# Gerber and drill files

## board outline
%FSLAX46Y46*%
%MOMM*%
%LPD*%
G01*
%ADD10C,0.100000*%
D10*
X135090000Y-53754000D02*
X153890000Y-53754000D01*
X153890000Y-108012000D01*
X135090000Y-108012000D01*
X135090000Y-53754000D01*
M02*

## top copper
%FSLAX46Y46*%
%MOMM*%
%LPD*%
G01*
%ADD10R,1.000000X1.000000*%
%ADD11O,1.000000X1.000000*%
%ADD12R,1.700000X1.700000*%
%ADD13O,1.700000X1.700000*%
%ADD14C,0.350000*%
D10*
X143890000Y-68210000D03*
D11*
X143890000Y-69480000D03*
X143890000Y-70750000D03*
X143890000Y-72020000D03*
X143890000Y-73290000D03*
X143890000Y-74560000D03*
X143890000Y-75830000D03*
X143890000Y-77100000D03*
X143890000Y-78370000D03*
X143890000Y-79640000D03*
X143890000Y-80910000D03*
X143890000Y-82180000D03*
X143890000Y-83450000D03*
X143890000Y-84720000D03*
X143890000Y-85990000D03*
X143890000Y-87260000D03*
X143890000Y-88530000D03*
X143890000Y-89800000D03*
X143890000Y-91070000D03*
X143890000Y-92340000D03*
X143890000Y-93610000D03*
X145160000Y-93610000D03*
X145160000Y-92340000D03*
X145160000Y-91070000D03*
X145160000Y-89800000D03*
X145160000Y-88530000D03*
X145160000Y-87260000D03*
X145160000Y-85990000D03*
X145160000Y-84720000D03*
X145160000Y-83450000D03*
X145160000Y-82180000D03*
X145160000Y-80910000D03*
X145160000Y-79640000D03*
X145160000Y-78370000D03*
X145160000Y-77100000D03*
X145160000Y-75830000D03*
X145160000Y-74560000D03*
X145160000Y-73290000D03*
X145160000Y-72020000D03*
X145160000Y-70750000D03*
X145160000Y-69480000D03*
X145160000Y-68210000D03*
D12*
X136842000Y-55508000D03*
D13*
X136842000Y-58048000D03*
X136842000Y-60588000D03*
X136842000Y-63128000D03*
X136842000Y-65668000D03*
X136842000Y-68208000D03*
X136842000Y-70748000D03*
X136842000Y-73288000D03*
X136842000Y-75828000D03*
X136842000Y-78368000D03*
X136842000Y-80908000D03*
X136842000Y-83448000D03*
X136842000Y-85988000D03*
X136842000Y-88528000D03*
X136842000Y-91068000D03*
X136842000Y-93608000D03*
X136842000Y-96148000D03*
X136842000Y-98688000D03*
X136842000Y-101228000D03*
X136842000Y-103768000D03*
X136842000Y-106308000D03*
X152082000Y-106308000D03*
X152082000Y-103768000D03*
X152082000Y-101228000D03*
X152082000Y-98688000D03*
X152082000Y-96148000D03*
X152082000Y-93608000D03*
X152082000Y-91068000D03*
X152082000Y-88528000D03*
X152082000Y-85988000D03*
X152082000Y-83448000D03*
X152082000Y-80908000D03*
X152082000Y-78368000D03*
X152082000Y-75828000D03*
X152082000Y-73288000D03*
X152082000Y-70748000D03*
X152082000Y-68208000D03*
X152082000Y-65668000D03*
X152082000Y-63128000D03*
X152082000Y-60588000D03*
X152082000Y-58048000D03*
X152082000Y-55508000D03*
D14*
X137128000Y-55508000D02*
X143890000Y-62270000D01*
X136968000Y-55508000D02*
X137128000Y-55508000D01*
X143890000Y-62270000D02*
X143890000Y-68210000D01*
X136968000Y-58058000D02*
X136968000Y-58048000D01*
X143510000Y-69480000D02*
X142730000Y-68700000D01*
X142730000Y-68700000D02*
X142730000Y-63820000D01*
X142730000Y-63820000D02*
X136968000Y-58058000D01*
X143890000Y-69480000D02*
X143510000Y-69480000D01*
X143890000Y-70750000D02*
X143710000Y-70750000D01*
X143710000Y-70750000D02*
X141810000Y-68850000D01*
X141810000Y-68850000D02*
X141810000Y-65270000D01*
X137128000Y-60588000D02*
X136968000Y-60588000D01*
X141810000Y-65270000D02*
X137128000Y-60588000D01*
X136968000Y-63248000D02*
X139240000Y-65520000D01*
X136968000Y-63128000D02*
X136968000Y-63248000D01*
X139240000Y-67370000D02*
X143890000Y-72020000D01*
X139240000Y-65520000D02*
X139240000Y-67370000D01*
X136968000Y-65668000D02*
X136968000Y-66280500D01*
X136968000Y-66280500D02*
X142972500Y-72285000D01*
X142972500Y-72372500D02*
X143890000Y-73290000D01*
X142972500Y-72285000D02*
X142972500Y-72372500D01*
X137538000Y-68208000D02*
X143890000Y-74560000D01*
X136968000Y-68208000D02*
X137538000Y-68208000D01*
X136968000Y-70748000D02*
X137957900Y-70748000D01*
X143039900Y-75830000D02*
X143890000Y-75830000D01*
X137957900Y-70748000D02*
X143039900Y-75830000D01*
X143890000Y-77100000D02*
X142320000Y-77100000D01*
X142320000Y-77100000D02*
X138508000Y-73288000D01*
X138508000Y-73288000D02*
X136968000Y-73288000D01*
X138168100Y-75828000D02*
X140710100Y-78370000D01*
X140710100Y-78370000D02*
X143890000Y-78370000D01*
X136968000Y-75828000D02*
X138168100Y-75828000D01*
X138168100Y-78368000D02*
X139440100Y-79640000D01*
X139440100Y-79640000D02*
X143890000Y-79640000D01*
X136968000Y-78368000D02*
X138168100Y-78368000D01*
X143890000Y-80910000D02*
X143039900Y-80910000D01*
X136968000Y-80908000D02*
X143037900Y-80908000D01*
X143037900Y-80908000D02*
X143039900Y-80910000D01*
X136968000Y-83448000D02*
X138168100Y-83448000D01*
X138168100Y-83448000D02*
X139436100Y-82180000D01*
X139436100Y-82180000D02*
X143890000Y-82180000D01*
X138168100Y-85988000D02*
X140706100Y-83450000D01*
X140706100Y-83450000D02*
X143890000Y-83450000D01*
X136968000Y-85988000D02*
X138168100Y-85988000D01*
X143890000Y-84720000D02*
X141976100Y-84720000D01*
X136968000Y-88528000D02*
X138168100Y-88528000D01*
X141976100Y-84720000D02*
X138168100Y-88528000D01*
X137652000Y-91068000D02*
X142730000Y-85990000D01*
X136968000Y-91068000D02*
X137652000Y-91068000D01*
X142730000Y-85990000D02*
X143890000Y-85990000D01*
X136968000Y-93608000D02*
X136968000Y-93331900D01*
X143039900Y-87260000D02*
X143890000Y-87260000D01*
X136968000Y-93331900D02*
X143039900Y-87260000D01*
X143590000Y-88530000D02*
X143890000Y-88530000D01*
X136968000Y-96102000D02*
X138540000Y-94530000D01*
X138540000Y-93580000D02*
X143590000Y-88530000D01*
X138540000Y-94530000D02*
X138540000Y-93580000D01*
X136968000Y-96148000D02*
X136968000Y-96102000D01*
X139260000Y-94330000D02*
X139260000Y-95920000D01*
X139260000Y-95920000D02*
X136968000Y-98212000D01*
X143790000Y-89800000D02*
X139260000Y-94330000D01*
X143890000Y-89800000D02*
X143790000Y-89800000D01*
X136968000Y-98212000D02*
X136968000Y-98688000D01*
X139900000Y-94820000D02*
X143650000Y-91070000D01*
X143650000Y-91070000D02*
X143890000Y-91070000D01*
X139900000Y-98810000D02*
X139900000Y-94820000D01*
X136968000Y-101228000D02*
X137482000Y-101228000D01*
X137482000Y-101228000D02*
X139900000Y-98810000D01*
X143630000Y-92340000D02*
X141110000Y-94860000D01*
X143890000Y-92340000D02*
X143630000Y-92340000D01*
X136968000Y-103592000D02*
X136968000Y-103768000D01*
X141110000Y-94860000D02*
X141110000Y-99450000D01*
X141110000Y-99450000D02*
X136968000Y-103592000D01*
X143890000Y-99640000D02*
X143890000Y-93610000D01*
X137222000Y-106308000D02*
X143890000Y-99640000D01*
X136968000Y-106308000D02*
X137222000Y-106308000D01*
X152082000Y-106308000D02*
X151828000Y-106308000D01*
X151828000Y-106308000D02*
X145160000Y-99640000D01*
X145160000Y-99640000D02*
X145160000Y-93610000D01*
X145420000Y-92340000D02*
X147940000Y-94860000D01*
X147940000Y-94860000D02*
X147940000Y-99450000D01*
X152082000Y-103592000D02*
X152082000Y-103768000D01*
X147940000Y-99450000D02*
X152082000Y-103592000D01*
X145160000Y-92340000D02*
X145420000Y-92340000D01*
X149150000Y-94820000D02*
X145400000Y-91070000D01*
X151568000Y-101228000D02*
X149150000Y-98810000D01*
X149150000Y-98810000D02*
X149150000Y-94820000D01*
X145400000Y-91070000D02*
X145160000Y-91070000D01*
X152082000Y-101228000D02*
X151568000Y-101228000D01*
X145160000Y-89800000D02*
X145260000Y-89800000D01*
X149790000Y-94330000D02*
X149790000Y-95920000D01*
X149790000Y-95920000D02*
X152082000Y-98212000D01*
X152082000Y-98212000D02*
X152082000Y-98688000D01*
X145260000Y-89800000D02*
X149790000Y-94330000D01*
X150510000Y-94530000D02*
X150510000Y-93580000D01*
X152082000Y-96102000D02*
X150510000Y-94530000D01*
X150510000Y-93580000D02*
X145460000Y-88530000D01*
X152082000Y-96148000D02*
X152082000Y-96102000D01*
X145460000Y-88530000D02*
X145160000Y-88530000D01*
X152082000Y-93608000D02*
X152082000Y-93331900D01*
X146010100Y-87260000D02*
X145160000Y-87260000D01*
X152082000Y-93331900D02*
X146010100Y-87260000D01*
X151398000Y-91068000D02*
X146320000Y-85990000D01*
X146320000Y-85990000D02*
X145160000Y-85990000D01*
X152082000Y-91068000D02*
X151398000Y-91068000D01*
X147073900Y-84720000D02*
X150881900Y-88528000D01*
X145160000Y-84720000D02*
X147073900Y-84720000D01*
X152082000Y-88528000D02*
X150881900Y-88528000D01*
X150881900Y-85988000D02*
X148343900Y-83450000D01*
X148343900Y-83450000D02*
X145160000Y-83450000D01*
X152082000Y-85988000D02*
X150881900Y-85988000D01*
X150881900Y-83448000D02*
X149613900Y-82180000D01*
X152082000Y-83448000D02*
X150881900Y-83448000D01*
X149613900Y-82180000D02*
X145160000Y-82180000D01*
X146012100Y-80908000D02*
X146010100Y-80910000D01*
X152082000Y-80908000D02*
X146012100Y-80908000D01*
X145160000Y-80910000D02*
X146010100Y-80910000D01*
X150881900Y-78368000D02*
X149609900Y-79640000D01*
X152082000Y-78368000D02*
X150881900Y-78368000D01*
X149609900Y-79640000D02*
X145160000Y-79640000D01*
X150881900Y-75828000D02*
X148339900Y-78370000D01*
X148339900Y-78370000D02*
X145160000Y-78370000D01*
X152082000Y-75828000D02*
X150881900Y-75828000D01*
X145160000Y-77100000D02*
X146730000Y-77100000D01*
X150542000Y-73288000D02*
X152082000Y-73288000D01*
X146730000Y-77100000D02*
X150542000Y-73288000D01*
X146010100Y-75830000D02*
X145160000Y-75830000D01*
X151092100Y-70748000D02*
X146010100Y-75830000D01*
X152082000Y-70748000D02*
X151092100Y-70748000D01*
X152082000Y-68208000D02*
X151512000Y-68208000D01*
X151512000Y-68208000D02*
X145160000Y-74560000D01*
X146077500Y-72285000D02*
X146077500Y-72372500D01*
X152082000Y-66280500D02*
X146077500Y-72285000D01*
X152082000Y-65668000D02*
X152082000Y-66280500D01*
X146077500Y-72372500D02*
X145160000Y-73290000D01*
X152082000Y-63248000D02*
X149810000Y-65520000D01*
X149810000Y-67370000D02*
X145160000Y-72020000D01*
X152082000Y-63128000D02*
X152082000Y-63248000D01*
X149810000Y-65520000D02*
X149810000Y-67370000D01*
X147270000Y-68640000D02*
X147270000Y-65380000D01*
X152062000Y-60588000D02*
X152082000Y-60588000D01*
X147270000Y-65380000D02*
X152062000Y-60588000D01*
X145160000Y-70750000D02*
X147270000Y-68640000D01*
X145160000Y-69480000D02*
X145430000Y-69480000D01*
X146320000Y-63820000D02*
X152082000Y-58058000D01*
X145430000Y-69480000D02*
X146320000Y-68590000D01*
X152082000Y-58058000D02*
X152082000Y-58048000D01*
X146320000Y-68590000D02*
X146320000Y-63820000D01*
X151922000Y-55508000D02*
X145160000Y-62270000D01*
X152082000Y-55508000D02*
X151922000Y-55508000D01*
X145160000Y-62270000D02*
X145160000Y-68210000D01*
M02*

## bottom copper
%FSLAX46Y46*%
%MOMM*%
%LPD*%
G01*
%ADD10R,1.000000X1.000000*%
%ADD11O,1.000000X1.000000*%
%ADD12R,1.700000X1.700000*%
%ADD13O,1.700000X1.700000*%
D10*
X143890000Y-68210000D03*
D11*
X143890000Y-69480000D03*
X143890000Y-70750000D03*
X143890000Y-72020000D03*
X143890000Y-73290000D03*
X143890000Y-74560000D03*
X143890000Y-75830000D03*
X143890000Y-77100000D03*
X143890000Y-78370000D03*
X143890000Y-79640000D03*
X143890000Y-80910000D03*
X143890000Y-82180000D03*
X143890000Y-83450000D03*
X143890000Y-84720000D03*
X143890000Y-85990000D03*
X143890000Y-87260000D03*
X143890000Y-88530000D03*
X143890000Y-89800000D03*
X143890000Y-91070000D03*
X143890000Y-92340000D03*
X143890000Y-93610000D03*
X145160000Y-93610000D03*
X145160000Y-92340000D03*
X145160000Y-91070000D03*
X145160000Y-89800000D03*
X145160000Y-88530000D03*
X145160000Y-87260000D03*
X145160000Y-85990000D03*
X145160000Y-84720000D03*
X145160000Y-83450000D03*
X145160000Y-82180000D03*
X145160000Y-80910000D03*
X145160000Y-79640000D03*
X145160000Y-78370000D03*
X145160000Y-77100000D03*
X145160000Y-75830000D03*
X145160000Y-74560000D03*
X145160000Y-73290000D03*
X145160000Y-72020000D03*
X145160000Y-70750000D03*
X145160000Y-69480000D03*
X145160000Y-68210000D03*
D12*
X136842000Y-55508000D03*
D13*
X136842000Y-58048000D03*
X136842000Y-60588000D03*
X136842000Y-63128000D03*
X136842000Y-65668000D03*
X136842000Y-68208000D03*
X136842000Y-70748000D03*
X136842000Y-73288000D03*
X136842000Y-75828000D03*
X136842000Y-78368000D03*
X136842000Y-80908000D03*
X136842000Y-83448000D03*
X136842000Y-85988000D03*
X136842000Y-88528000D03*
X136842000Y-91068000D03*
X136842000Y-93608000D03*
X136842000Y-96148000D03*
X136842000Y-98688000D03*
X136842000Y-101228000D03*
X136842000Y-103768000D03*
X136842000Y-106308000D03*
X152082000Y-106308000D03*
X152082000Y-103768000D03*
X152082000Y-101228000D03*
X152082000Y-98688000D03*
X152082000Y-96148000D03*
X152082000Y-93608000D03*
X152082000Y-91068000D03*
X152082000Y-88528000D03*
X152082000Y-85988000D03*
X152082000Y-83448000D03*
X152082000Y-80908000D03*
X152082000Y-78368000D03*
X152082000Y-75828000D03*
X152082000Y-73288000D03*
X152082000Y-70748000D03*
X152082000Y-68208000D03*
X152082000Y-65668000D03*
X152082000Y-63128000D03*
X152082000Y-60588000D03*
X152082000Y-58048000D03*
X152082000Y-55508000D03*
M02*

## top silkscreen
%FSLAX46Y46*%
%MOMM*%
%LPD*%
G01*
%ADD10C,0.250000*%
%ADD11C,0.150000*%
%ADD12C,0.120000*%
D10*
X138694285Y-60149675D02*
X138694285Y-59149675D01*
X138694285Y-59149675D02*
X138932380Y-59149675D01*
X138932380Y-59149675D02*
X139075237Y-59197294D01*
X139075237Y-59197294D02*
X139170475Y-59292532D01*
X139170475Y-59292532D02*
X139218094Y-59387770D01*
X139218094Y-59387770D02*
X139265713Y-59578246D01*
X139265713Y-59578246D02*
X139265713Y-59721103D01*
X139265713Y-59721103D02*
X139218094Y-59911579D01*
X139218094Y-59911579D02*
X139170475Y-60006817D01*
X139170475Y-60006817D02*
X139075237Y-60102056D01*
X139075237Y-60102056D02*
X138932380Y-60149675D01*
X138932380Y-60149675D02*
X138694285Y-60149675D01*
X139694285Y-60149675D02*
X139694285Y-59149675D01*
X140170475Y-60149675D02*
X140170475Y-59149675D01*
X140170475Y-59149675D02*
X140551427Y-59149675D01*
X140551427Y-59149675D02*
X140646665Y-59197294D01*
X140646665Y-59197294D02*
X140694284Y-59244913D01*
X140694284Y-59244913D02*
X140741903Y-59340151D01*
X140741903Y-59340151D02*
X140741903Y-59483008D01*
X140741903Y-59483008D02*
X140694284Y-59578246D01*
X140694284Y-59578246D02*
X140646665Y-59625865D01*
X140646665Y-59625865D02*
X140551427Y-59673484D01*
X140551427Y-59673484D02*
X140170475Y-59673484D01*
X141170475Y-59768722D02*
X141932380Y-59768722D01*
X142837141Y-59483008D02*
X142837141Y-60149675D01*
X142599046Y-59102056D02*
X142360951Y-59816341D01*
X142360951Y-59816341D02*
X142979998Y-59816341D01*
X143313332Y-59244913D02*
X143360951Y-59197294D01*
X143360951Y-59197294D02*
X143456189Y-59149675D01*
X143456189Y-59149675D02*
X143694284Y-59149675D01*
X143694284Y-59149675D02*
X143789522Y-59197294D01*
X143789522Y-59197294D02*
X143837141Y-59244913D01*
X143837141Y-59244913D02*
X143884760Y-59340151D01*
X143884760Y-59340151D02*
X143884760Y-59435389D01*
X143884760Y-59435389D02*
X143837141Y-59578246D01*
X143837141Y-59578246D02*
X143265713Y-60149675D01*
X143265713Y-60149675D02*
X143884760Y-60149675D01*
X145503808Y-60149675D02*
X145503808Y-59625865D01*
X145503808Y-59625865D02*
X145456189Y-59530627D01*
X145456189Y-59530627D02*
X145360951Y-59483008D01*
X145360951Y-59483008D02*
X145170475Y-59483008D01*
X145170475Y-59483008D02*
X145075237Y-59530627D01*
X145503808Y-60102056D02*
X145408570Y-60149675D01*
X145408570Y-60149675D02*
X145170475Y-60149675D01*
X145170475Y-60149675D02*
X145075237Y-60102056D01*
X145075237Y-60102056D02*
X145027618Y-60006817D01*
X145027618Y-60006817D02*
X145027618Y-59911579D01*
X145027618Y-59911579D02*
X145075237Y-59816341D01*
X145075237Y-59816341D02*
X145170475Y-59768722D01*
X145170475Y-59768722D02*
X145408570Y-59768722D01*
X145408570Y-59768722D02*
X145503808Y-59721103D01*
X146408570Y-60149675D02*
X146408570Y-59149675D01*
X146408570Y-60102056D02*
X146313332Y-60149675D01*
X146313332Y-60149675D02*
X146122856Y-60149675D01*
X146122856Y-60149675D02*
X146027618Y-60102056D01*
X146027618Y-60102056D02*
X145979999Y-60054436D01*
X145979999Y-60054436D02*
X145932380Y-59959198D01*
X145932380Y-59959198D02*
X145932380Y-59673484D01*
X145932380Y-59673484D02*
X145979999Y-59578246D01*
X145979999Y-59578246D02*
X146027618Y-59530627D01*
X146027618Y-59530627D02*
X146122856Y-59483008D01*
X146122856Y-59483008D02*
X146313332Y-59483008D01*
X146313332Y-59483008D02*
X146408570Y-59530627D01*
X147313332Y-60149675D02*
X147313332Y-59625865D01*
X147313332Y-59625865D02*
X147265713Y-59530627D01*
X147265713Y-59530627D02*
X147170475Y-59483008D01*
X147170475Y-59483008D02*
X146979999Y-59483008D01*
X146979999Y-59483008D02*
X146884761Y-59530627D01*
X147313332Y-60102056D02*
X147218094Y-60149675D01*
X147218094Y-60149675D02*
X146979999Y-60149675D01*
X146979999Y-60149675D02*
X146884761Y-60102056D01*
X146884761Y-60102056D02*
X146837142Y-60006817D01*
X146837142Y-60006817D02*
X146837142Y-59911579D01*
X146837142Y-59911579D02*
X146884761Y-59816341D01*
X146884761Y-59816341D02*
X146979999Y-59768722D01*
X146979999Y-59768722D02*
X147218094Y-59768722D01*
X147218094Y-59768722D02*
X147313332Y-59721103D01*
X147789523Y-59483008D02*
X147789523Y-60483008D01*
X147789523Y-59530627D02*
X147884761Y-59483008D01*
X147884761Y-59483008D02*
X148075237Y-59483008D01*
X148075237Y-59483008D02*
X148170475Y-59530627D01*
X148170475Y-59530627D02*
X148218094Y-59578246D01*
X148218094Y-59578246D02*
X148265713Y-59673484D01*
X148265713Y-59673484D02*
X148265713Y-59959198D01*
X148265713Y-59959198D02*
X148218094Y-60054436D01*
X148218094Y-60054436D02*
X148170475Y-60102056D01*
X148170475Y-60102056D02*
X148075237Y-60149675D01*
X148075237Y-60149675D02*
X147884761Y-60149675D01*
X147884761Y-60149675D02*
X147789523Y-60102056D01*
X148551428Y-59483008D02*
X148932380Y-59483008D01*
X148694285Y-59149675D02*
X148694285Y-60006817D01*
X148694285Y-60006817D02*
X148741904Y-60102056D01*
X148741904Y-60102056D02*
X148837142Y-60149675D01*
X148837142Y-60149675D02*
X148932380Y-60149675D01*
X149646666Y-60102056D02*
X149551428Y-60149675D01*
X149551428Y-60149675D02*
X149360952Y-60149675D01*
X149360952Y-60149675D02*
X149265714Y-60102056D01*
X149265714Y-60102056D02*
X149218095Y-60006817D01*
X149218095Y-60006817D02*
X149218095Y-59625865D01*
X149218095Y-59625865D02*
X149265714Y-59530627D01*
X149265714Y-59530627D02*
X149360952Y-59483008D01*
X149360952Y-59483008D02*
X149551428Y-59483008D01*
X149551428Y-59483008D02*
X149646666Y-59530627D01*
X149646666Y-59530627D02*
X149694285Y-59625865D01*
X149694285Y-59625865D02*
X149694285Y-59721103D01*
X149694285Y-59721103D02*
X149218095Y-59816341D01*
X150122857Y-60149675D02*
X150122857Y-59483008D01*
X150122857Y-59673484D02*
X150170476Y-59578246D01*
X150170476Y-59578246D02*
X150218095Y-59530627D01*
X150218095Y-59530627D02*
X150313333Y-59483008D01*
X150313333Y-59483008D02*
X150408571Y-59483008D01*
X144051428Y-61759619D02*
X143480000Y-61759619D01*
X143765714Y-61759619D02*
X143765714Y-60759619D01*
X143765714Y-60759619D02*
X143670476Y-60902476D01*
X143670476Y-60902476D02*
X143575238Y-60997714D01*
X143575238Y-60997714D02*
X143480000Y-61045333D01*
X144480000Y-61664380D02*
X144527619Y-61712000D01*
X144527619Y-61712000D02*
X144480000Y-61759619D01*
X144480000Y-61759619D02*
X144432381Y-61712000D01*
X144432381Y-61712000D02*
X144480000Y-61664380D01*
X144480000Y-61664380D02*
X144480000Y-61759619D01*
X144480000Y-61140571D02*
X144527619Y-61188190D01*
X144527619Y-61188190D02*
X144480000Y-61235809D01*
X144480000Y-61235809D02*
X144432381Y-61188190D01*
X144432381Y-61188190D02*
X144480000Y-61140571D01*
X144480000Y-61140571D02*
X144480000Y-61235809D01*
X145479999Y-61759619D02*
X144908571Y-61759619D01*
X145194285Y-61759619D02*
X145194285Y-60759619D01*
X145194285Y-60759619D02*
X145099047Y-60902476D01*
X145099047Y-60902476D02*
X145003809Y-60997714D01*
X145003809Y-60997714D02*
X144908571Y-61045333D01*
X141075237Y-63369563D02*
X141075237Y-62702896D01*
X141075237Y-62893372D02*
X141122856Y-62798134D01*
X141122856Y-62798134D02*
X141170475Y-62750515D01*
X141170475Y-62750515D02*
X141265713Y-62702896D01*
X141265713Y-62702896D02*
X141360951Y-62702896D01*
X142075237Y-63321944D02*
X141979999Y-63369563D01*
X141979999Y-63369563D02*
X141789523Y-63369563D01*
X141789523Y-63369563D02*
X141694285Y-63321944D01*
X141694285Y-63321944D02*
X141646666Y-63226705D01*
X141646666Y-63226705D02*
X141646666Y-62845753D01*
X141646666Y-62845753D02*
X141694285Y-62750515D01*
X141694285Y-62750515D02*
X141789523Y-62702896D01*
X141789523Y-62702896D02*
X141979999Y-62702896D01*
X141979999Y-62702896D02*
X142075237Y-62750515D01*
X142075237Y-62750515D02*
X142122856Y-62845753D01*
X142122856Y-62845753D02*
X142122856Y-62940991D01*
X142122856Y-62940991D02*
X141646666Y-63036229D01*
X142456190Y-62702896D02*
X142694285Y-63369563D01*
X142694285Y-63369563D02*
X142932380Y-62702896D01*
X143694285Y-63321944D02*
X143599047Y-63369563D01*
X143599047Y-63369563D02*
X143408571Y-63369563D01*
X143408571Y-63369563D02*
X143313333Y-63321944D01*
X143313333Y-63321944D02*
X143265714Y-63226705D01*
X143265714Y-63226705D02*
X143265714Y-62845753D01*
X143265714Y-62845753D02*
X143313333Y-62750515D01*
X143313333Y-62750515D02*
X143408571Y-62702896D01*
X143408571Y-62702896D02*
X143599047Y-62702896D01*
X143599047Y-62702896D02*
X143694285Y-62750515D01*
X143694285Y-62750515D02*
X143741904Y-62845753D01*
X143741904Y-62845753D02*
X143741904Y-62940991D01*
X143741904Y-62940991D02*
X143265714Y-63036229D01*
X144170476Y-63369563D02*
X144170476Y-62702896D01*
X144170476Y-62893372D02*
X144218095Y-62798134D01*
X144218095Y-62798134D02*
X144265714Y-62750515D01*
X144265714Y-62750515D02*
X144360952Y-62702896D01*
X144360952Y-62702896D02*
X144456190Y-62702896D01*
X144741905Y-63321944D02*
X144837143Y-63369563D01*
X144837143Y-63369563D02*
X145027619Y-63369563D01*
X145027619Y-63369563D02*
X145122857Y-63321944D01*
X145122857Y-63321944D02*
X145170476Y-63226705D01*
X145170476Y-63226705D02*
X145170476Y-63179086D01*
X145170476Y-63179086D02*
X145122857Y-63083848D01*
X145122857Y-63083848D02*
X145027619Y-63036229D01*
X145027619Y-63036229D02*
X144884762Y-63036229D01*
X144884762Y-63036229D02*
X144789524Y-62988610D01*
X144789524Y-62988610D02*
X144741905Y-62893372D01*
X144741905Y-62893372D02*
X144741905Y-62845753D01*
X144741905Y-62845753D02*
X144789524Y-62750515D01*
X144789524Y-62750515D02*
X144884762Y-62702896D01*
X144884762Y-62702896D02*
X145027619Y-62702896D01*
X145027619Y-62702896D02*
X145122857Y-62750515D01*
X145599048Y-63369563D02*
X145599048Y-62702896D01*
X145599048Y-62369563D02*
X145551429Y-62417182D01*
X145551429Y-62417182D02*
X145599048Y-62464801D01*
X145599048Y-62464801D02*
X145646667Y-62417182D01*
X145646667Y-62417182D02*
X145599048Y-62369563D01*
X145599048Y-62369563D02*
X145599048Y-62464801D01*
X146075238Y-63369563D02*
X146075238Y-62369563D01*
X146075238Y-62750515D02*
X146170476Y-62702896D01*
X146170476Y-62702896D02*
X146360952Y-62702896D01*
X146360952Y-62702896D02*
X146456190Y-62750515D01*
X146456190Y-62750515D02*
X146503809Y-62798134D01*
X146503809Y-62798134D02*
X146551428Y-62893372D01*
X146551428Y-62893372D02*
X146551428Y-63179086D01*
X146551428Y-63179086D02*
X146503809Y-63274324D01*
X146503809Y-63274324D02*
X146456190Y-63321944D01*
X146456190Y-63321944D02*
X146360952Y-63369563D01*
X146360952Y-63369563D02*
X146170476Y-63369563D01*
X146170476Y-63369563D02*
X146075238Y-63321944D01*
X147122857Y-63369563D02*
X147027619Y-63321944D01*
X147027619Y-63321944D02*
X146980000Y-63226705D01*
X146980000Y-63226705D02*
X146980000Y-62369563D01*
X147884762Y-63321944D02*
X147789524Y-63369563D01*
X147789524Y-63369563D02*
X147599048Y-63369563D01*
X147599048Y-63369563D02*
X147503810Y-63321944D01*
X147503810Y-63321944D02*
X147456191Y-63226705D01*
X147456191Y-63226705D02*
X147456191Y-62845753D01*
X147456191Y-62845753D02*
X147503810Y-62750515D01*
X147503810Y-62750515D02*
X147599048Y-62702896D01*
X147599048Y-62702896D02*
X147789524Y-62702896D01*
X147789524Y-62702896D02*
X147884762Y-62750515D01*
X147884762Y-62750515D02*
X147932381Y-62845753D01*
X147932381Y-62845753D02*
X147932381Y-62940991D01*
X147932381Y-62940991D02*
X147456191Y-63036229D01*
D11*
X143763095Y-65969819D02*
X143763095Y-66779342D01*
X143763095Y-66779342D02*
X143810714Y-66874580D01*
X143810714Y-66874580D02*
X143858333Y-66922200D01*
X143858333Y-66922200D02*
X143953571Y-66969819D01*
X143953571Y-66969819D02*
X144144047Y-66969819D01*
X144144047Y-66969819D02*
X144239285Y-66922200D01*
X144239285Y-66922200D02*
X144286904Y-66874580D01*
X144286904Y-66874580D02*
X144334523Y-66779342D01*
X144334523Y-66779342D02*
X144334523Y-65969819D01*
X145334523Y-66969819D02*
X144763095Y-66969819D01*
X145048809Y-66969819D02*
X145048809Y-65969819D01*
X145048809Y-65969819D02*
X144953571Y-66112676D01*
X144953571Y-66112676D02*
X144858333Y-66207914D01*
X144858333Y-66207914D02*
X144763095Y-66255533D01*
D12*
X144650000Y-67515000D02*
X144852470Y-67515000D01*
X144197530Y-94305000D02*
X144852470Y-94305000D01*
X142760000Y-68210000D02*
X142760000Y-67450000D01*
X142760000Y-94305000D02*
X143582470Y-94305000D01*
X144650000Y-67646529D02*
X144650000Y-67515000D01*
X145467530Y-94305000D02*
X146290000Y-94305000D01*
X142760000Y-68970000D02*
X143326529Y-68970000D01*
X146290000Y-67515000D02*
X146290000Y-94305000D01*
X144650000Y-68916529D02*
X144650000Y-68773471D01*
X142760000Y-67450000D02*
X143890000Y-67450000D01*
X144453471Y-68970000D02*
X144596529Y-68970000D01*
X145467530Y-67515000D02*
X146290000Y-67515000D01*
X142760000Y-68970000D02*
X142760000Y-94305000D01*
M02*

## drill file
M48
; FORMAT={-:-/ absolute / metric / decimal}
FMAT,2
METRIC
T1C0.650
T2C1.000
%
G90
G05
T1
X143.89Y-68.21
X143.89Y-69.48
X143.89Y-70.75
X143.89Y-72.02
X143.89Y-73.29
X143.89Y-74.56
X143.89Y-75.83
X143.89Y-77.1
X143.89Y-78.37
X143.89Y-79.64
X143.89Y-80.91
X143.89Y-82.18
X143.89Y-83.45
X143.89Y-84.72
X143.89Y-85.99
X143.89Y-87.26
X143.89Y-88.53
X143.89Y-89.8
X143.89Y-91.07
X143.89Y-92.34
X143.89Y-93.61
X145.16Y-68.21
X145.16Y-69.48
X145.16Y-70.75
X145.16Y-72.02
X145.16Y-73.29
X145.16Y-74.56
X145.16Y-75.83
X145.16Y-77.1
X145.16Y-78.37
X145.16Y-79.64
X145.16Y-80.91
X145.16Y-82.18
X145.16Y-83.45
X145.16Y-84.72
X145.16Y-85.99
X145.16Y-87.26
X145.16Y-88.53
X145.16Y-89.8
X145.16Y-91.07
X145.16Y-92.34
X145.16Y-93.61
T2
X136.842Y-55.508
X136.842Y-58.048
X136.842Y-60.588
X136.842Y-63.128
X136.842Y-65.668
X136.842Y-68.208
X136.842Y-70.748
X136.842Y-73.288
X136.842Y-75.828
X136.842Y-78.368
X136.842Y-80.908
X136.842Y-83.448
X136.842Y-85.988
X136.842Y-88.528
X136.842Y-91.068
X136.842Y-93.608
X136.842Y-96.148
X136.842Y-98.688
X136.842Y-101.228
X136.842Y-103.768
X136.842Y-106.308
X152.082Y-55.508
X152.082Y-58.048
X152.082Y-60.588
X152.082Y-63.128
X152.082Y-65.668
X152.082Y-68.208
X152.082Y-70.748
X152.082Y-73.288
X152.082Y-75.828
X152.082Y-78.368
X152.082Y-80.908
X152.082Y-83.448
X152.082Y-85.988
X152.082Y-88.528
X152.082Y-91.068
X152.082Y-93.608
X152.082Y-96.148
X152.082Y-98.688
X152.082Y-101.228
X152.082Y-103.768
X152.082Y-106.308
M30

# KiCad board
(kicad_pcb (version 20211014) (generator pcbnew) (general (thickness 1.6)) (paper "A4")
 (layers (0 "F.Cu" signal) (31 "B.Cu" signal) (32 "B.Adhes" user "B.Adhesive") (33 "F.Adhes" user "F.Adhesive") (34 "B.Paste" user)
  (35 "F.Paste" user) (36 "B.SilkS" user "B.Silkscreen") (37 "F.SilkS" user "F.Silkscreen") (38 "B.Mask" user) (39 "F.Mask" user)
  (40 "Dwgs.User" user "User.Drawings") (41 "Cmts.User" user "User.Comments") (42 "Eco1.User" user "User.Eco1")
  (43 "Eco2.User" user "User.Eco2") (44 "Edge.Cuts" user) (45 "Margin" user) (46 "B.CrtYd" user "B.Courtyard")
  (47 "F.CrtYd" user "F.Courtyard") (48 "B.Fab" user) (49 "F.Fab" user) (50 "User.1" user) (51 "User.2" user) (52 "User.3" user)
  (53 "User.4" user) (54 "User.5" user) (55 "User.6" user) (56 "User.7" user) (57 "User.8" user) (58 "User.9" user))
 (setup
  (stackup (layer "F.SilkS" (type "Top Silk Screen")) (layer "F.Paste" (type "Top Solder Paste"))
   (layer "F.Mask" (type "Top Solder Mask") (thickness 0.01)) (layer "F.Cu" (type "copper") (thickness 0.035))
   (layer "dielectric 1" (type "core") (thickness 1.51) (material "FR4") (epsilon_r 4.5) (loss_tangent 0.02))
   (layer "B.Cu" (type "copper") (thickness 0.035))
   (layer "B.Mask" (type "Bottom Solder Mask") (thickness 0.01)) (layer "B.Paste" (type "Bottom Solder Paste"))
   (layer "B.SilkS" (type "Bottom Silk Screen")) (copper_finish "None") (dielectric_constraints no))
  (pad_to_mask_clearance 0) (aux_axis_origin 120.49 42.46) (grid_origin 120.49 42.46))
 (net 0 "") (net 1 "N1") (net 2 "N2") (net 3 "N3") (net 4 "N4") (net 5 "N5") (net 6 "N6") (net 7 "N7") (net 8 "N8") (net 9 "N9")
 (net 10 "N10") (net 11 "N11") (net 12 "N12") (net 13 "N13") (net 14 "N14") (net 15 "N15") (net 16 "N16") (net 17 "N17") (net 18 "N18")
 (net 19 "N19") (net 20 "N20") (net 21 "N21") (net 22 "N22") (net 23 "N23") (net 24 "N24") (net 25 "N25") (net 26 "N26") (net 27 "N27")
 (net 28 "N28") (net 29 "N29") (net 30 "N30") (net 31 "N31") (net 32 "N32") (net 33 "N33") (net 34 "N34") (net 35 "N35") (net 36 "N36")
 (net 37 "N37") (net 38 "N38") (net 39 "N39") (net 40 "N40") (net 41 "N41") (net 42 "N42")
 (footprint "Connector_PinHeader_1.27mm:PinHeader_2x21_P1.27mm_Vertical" (layer "F.Cu") (at 143.89 68.21)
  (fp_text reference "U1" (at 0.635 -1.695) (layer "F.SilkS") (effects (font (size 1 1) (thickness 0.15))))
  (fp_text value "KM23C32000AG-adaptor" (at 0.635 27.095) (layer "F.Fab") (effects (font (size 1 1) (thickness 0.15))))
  (fp_line (start 0.76 -0.695) (end 0.96247 -0.695) (layer "F.SilkS") (width 0.12))
  (fp_line (start 0.30753 26.095) (end 0.96247 26.095) (layer "F.SilkS") (width 0.12))
  (fp_line (start -1.13 0) (end -1.13 -0.76) (layer "F.SilkS") (width 0.12))
  (fp_line (start -1.13 26.095) (end -0.30753 26.095) (layer "F.SilkS") (width 0.12))
  (fp_line (start 0.76 -0.563471) (end 0.76 -0.695) (layer "F.SilkS") (width 0.12))
  (fp_line (start 1.57753 26.095) (end 2.4 26.095) (layer "F.SilkS") (width 0.12))
  (fp_line (start -1.13 0.76) (end -0.563471 0.76) (layer "F.SilkS") (width 0.12))
  (fp_line (start 2.4 -0.695) (end 2.4 26.095) (layer "F.SilkS") (width 0.12))
  (fp_line (start 0.76 0.706529) (end 0.76 0.563471) (layer "F.SilkS") (width 0.12))
  (fp_line (start -1.13 -0.76) (end 0 -0.76) (layer "F.SilkS") (width 0.12))
  (fp_line (start 0.563471 0.76) (end 0.706529 0.76) (layer "F.SilkS") (width 0.12))
  (fp_line (start 1.57753 -0.695) (end 2.4 -0.695) (layer "F.SilkS") (width 0.12))
  (fp_line (start -1.13 0.76) (end -1.13 26.095) (layer "F.SilkS") (width 0.12))
  (pad "1" thru_hole rect (at 0 0) (size 1 1) (drill 0.65) (layers *.Cu *.Mask) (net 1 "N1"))
  (pad "2" thru_hole oval (at 0 1.27) (size 1 1) (drill 0.65) (layers *.Cu *.Mask) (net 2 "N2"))
  (pad "3" thru_hole oval (at 0 2.54) (size 1 1) (drill 0.65) (layers *.Cu *.Mask) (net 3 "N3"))
  (pad "4" thru_hole oval (at 0 3.81) (size 1 1) (drill 0.65) (layers *.Cu *.Mask) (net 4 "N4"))
  (pad "5" thru_hole oval (at 0 5.08) (size 1 1) (drill 0.65) (layers *.Cu *.Mask) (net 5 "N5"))
  (pad "6" thru_hole oval (at 0 6.35) (size 1 1) (drill 0.65) (layers *.Cu *.Mask) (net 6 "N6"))
  (pad "7" thru_hole oval (at 0 7.62) (size 1 1) (drill 0.65) (layers *.Cu *.Mask) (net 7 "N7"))
  (pad "8" thru_hole oval (at 0 8.89) (size 1 1) (drill 0.65) (layers *.Cu *.Mask) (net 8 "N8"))
  (pad "9" thru_hole oval (at 0 10.16) (size 1 1) (drill 0.65) (layers *.Cu *.Mask) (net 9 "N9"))
  (pad "10" thru_hole oval (at 0 11.43) (size 1 1) (drill 0.65) (layers *.Cu *.Mask) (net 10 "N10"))
  (pad "11" thru_hole oval (at 0 12.7) (size 1 1) (drill 0.65) (layers *.Cu *.Mask) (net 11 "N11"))
  (pad "12" thru_hole oval (at 0 13.97) (size 1 1) (drill 0.65) (layers *.Cu *.Mask) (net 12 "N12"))
  (pad "13" thru_hole oval (at 0 15.24) (size 1 1) (drill 0.65) (layers *.Cu *.Mask) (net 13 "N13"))
  (pad "14" thru_hole oval (at 0 16.51) (size 1 1) (drill 0.65) (layers *.Cu *.Mask) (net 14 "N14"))
  (pad "15" thru_hole oval (at 0 17.78) (size 1 1) (drill 0.65) (layers *.Cu *.Mask) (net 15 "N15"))
  (pad "16" thru_hole oval (at 0 19.05) (size 1 1) (drill 0.65) (layers *.Cu *.Mask) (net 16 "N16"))
  (pad "17" thru_hole oval (at 0 20.32) (size 1 1) (drill 0.65) (layers *.Cu *.Mask) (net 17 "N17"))
  (pad "18" thru_hole oval (at 0 21.59) (size 1 1) (drill 0.65) (layers *.Cu *.Mask) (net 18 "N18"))
  (pad "19" thru_hole oval (at 0 22.86) (size 1 1) (drill 0.65) (layers *.Cu *.Mask) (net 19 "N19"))
  (pad "20" thru_hole oval (at 0 24.13) (size 1 1) (drill 0.65) (layers *.Cu *.Mask) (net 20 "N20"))
  (pad "21" thru_hole oval (at 0 25.4) (size 1 1) (drill 0.65) (layers *.Cu *.Mask) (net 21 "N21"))
  (pad "22" thru_hole oval (at 1.27 25.4) (size 1 1) (drill 0.65) (layers *.Cu *.Mask) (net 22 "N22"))
  (pad "23" thru_hole oval (at 1.27 24.13) (size 1 1) (drill 0.65) (layers *.Cu *.Mask) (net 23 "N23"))
  (pad "24" thru_hole oval (at 1.27 22.86) (size 1 1) (drill 0.65) (layers *.Cu *.Mask) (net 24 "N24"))
  (pad "25" thru_hole oval (at 1.27 21.59) (size 1 1) (drill 0.65) (layers *.Cu *.Mask) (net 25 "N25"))
  (pad "26" thru_hole oval (at 1.27 20.32) (size 1 1) (drill 0.65) (layers *.Cu *.Mask) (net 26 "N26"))
  (pad "27" thru_hole oval (at 1.27 19.05) (size 1 1) (drill 0.65) (layers *.Cu *.Mask) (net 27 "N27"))
  (pad "28" thru_hole oval (at 1.27 17.78) (size 1 1) (drill 0.65) (layers *.Cu *.Mask) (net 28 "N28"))
  (pad "29" thru_hole oval (at 1.27 16.51) (size 1 1) (drill 0.65) (layers *.Cu *.Mask) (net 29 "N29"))
  (pad "30" thru_hole oval (at 1.27 15.24) (size 1 1) (drill 0.65) (layers *.Cu *.Mask) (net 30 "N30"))
  (pad "31" thru_hole oval (at 1.27 13.97) (size 1 1) (drill 0.65) (layers *.Cu *.Mask) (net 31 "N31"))
  (pad "32" thru_hole oval (at 1.27 12.7) (size 1 1) (drill 0.65) (layers *.Cu *.Mask) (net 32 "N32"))
  (pad "33" thru_hole oval (at 1.27 11.43) (size 1 1) (drill 0.65) (layers *.Cu *.Mask) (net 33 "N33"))
  (pad "34" thru_hole oval (at 1.27 10.16) (size 1 1) (drill 0.65) (layers *.Cu *.Mask) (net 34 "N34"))
  (pad "35" thru_hole oval (at 1.27 8.89) (size 1 1) (drill 0.65) (layers *.Cu *.Mask) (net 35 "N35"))
  (pad "36" thru_hole oval (at 1.27 7.62) (size 1 1) (drill 0.65) (layers *.Cu *.Mask) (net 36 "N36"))
  (pad "37" thru_hole oval (at 1.27 6.35) (size 1 1) (drill 0.65) (layers *.Cu *.Mask) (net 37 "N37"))
  (pad "38" thru_hole oval (at 1.27 5.08) (size 1 1) (drill 0.65) (layers *.Cu *.Mask) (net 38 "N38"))
  (pad "39" thru_hole oval (at 1.27 3.81) (size 1 1) (drill 0.65) (layers *.Cu *.Mask) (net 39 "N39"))
  (pad "40" thru_hole oval (at 1.27 2.54) (size 1 1) (drill 0.65) (layers *.Cu *.Mask) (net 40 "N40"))
  (pad "41" thru_hole oval (at 1.27 1.27) (size 1 1) (drill 0.65) (layers *.Cu *.Mask) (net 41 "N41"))
  (pad "42" thru_hole oval (at 1.27 0) (size 1 1) (drill 0.65) (layers *.Cu *.Mask) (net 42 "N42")))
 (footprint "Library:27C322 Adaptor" (layer "B.Cu") (at 152.082 55.508 180)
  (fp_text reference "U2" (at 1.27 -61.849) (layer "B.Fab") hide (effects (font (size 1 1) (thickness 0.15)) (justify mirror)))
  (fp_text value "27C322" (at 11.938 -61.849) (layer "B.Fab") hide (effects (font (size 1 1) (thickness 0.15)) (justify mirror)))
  (pad "1" thru_hole rect (at 15.24 0 180) (size 1.7 1.7) (drill 1) (layers *.Cu *.Mask) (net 1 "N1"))
  (pad "2" thru_hole oval (at 15.24 -2.54 180) (size 1.7 1.7) (drill 1) (layers *.Cu *.Mask) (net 2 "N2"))
  (pad "3" thru_hole oval (at 15.24 -5.08 180) (size 1.7 1.7) (drill 1) (layers *.Cu *.Mask) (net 3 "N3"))
  (pad "4" thru_hole oval (at 15.24 -7.62 180) (size 1.7 1.7) (drill 1) (layers *.Cu *.Mask) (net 4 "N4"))
  (pad "5" thru_hole oval (at 15.24 -10.16 180) (size 1.7 1.7) (drill 1) (layers *.Cu *.Mask) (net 5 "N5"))
  (pad "6" thru_hole oval (at 15.24 -12.7 180) (size 1.7 1.7) (drill 1) (layers *.Cu *.Mask) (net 6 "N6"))
  (pad "7" thru_hole oval (at 15.24 -15.24 180) (size 1.7 1.7) (drill 1) (layers *.Cu *.Mask) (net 7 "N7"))
  (pad "8" thru_hole oval (at 15.24 -17.78 180) (size 1.7 1.7) (drill 1) (layers *.Cu *.Mask) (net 8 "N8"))
  (pad "9" thru_hole oval (at 15.24 -20.32 180) (size 1.7 1.7) (drill 1) (layers *.Cu *.Mask) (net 9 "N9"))
  (pad "10" thru_hole oval (at 15.24 -22.86 180) (size 1.7 1.7) (drill 1) (layers *.Cu *.Mask) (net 10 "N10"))
  (pad "11" thru_hole oval (at 15.24 -25.4 180) (size 1.7 1.7) (drill 1) (layers *.Cu *.Mask) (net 11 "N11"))
  (pad "12" thru_hole oval (at 15.24 -27.94 180) (size 1.7 1.7) (drill 1) (layers *.Cu *.Mask) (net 12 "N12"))
  (pad "13" thru_hole oval (at 15.24 -30.48 180) (size 1.7 1.7) (drill 1) (layers *.Cu *.Mask) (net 13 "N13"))
  (pad "14" thru_hole oval (at 15.24 -33.02 180) (size 1.7 1.7) (drill 1) (layers *.Cu *.Mask) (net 14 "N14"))
  (pad "15" thru_hole oval (at 15.24 -35.56 180) (size 1.7 1.7) (drill 1) (layers *.Cu *.Mask) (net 15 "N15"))
  (pad "16" thru_hole oval (at 15.24 -38.1 180) (size 1.7 1.7) (drill 1) (layers *.Cu *.Mask) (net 16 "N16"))
  (pad "17" thru_hole oval (at 15.24 -40.64 180) (size 1.7 1.7) (drill 1) (layers *.Cu *.Mask) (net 17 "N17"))
  (pad "18" thru_hole oval (at 15.24 -43.18 180) (size 1.7 1.7) (drill 1) (layers *.Cu *.Mask) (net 18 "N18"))
  (pad "19" thru_hole oval (at 15.24 -45.72 180) (size 1.7 1.7) (drill 1) (layers *.Cu *.Mask) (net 19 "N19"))
  (pad "20" thru_hole oval (at 15.24 -48.26 180) (size 1.7 1.7) (drill 1) (layers *.Cu *.Mask) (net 20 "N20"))
  (pad "21" thru_hole oval (at 15.24 -50.8 180) (size 1.7 1.7) (drill 1) (layers *.Cu *.Mask) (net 21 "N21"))
  (pad "22" thru_hole oval (at 0 -50.8 180) (size 1.7 1.7) (drill 1) (layers *.Cu *.Mask) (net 22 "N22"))
  (pad "23" thru_hole oval (at 0 -48.26 180) (size 1.7 1.7) (drill 1) (layers *.Cu *.Mask) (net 23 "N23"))
  (pad "24" thru_hole oval (at 0 -45.72 180) (size 1.7 1.7) (drill 1) (layers *.Cu *.Mask) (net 24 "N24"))
  (pad "25" thru_hole oval (at 0 -43.18 180) (size 1.7 1.7) (drill 1) (layers *.Cu *.Mask) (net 25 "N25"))
  (pad "26" thru_hole oval (at 0 -40.64 180) (size 1.7 1.7) (drill 1) (layers *.Cu *.Mask) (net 26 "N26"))
  (pad "27" thru_hole oval (at 0 -38.1 180) (size 1.7 1.7) (drill 1) (layers *.Cu *.Mask) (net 27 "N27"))
  (pad "28" thru_hole oval (at 0 -35.56 180) (size 1.7 1.7) (drill 1) (layers *.Cu *.Mask) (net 28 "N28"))
  (pad "29" thru_hole oval (at 0 -33.02 180) (size 1.7 1.7) (drill 1) (layers *.Cu *.Mask) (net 29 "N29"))
  (pad "30" thru_hole oval (at 0 -30.48 180) (size 1.7 1.7) (drill 1) (layers *.Cu *.Mask) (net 30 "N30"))
  (pad "31" thru_hole oval (at 0 -27.94 180) (size 1.7 1.7) (drill 1) (layers *.Cu *.Mask) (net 31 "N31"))
  (pad "32" thru_hole oval (at 0 -25.4 180) (size 1.7 1.7) (drill 1) (layers *.Cu *.Mask) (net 32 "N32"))
  (pad "33" thru_hole oval (at 0 -22.86 180) (size 1.7 1.7) (drill 1) (layers *.Cu *.Mask) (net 33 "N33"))
  (pad "34" thru_hole oval (at 0 -20.32 180) (size 1.7 1.7) (drill 1) (layers *.Cu *.Mask) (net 34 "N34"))
  (pad "35" thru_hole oval (at 0 -17.78 180) (size 1.7 1.7) (drill 1) (layers *.Cu *.Mask) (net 35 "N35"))
  (pad "36" thru_hole oval (at 0 -15.24 180) (size 1.7 1.7) (drill 1) (layers *.Cu *.Mask) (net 36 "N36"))
  (pad "37" thru_hole oval (at 0 -12.7 180) (size 1.7 1.7) (drill 1) (layers *.Cu *.Mask) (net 37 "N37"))
  (pad "38" thru_hole oval (at 0 -10.16 180) (size 1.7 1.7) (drill 1) (layers *.Cu *.Mask) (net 38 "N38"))
  (pad "39" thru_hole oval (at 0 -7.62 180) (size 1.7 1.7) (drill 1) (layers *.Cu *.Mask) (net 39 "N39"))
  (pad "40" thru_hole oval (at 0 -5.08 180) (size 1.7 1.7) (drill 1) (layers *.Cu *.Mask) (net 40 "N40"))
  (pad "41" thru_hole oval (at 0 -2.54 180) (size 1.7 1.7) (drill 1) (layers *.Cu *.Mask) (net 41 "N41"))
  (pad "42" thru_hole oval (at 0 0 180) (size 1.7 1.7) (drill 1) (layers *.Cu *.Mask) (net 42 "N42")))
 (gr_rect (start 135.09 53.754) (end 153.89 108.012) (layer "Edge.Cuts") (width 0.1) (fill none))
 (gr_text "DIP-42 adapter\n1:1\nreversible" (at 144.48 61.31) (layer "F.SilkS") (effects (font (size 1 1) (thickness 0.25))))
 (segment (start 137.128 55.508) (end 143.89 62.27) (width 0.35) (layer "F.Cu") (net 1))
 (segment (start 136.968 55.508) (end 137.128 55.508) (width 0.35) (layer "F.Cu") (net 1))
 (segment (start 143.89 62.27) (end 143.89 68.21) (width 0.35) (layer "F.Cu") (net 1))
 (segment (start 136.968 58.058) (end 136.968 58.048) (width 0.35) (layer "F.Cu") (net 2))
 (segment (start 143.51 69.48) (end 142.73 68.7) (width 0.35) (layer "F.Cu") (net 2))
 (segment (start 142.73 68.7) (end 142.73 63.82) (width 0.35) (layer "F.Cu") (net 2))
 (segment (start 142.73 63.82) (end 136.968 58.058) (width 0.35) (layer "F.Cu") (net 2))
 (segment (start 143.89 69.48) (end 143.51 69.48) (width 0.35) (layer "F.Cu") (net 2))
 (segment (start 143.89 70.75) (end 143.71 70.75) (width 0.35) (layer "F.Cu") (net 3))
 (segment (start 143.71 70.75) (end 141.81 68.85) (width 0.35) (layer "F.Cu") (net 3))
 (segment (start 141.81 68.85) (end 141.81 65.27) (width 0.35) (layer "F.Cu") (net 3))
 (segment (start 137.128 60.588) (end 136.968 60.588) (width 0.35) (layer "F.Cu") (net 3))
 (segment (start 141.81 65.27) (end 137.128 60.588) (width 0.35) (layer "F.Cu") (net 3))
 (segment (start 136.968 63.248) (end 139.24 65.52) (width 0.35) (layer "F.Cu") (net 4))
 (segment (start 136.968 63.128) (end 136.968 63.248) (width 0.35) (layer "F.Cu") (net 4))
 (segment (start 139.24 67.37) (end 143.89 72.02) (width 0.35) (layer "F.Cu") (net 4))
 (segment (start 139.24 65.52) (end 139.24 67.37) (width 0.35) (layer "F.Cu") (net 4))
 (segment (start 136.968 65.668) (end 136.968 66.2805) (width 0.35) (layer "F.Cu") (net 5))
 (segment (start 136.968 66.2805) (end 142.9725 72.285) (width 0.35) (layer "F.Cu") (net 5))
 (segment (start 142.9725 72.3725) (end 143.89 73.29) (width 0.35) (layer "F.Cu") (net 5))
 (segment (start 142.9725 72.285) (end 142.9725 72.3725) (width 0.35) (layer "F.Cu") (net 5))
 (segment (start 137.538 68.208) (end 143.89 74.56) (width 0.35) (layer "F.Cu") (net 6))
 (segment (start 136.968 68.208) (end 137.538 68.208) (width 0.35) (layer "F.Cu") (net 6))
 (segment (start 136.968 70.748) (end 137.9579 70.748) (width 0.35) (layer "F.Cu") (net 7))
 (segment (start 143.0399 75.83) (end 143.89 75.83) (width 0.35) (layer "F.Cu") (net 7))
 (segment (start 137.9579 70.748) (end 143.0399 75.83) (width 0.35) (layer "F.Cu") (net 7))
 (segment (start 143.89 77.1) (end 142.32 77.1) (width 0.35) (layer "F.Cu") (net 8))
 (segment (start 142.32 77.1) (end 138.508 73.288) (width 0.35) (layer "F.Cu") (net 8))
 (segment (start 138.508 73.288) (end 136.968 73.288) (width 0.35) (layer "F.Cu") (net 8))
 (segment (start 138.1681 75.828) (end 140.7101 78.37) (width 0.35) (layer "F.Cu") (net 9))
 (segment (start 140.7101 78.37) (end 143.89 78.37) (width 0.35) (layer "F.Cu") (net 9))
 (segment (start 136.968 75.828) (end 138.1681 75.828) (width 0.35) (layer "F.Cu") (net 9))
 (segment (start 138.1681 78.368) (end 139.4401 79.64) (width 0.35) (layer "F.Cu") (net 10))
 (segment (start 139.4401 79.64) (end 143.89 79.64) (width 0.35) (layer "F.Cu") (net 10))
 (segment (start 136.968 78.368) (end 138.1681 78.368) (width 0.35) (layer "F.Cu") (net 10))
 (segment (start 143.89 80.91) (end 143.0399 80.91) (width 0.35) (layer "F.Cu") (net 11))
 (segment (start 136.968 80.908) (end 143.0379 80.908) (width 0.35) (layer "F.Cu") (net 11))
 (segment (start 143.0379 80.908) (end 143.0399 80.91) (width 0.35) (layer "F.Cu") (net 11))
 (segment (start 136.968 83.448) (end 138.1681 83.448) (width 0.35) (layer "F.Cu") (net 12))
 (segment (start 138.1681 83.448) (end 139.4361 82.18) (width 0.35) (layer "F.Cu") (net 12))
 (segment (start 139.4361 82.18) (end 143.89 82.18) (width 0.35) (layer "F.Cu") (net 12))
 (segment (start 138.1681 85.988) (end 140.7061 83.45) (width 0.35) (layer "F.Cu") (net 13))
 (segment (start 140.7061 83.45) (end 143.89 83.45) (width 0.35) (layer "F.Cu") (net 13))
 (segment (start 136.968 85.988) (end 138.1681 85.988) (width 0.35) (layer "F.Cu") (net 13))
 (segment (start 143.89 84.72) (end 141.9761 84.72) (width 0.35) (layer "F.Cu") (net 14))
 (segment (start 136.968 88.528) (end 138.1681 88.528) (width 0.35) (layer "F.Cu") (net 14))
 (segment (start 141.9761 84.72) (end 138.1681 88.528) (width 0.35) (layer "F.Cu") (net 14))
 (segment (start 137.652 91.068) (end 142.73 85.99) (width 0.35) (layer "F.Cu") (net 15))
 (segment (start 136.968 91.068) (end 137.652 91.068) (width 0.35) (layer "F.Cu") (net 15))
 (segment (start 142.73 85.99) (end 143.89 85.99) (width 0.35) (layer "F.Cu") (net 15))
 (segment (start 136.968 93.608) (end 136.968 93.3319) (width 0.35) (layer "F.Cu") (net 16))
 (segment (start 143.0399 87.26) (end 143.89 87.26) (width 0.35) (layer "F.Cu") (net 16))
 (segment (start 136.968 93.3319) (end 143.0399 87.26) (width 0.35) (layer "F.Cu") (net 16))
 (segment (start 143.59 88.53) (end 143.89 88.53) (width 0.35) (layer "F.Cu") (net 17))
 (segment (start 136.968 96.102) (end 138.54 94.53) (width 0.35) (layer "F.Cu") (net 17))
 (segment (start 138.54 93.58) (end 143.59 88.53) (width 0.35) (layer "F.Cu") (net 17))
 (segment (start 138.54 94.53) (end 138.54 93.58) (width 0.35) (layer "F.Cu") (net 17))
 (segment (start 136.968 96.148) (end 136.968 96.102) (width 0.35) (layer "F.Cu") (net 17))
 (segment (start 139.26 94.33) (end 139.26 95.92) (width 0.35) (layer "F.Cu") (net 18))
 (segment (start 139.26 95.92) (end 136.968 98.212) (width 0.35) (layer "F.Cu") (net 18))
 (segment (start 143.79 89.8) (end 139.26 94.33) (width 0.35) (layer "F.Cu") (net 18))
 (segment (start 143.89 89.8) (end 143.79 89.8) (width 0.35) (layer "F.Cu") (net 18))
 (segment (start 136.968 98.212) (end 136.968 98.688) (width 0.35) (layer "F.Cu") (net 18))
 (segment (start 139.9 94.82) (end 143.65 91.07) (width 0.35) (layer "F.Cu") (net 19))
 (segment (start 143.65 91.07) (end 143.89 91.07) (width 0.35) (layer "F.Cu") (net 19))
 (segment (start 139.9 98.81) (end 139.9 94.82) (width 0.35) (layer "F.Cu") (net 19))
 (segment (start 136.968 101.228) (end 137.482 101.228) (width 0.35) (layer "F.Cu") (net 19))
 (segment (start 137.482 101.228) (end 139.9 98.81) (width 0.35) (layer "F.Cu") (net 19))
 (segment (start 143.63 92.34) (end 141.11 94.86) (width 0.35) (layer "F.Cu") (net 20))
 (segment (start 143.89 92.34) (end 143.63 92.34) (width 0.35) (layer "F.Cu") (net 20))
 (segment (start 136.968 103.592) (end 136.968 103.768) (width 0.35) (layer "F.Cu") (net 20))
 (segment (start 141.11 94.86) (end 141.11 99.45) (width 0.35) (layer "F.Cu") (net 20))
 (segment (start 141.11 99.45) (end 136.968 103.592) (width 0.35) (layer "F.Cu") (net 20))
 (segment (start 143.89 99.64) (end 143.89 93.61) (width 0.35) (layer "F.Cu") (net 21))
 (segment (start 137.222 106.308) (end 143.89 99.64) (width 0.35) (layer "F.Cu") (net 21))
 (segment (start 136.968 106.308) (end 137.222 106.308) (width 0.35) (layer "F.Cu") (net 21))
 (segment (start 152.082 106.308) (end 151.828 106.308) (width 0.35) (layer "F.Cu") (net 22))
 (segment (start 151.828 106.308) (end 145.16 99.64) (width 0.35) (layer "F.Cu") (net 22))
 (segment (start 145.16 99.64) (end 145.16 93.61) (width 0.35) (layer "F.Cu") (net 22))
 (segment (start 145.42 92.34) (end 147.94 94.86) (width 0.35) (layer "F.Cu") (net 23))
 (segment (start 147.94 94.86) (end 147.94 99.45) (width 0.35) (layer "F.Cu") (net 23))
 (segment (start 152.082 103.592) (end 152.082 103.768) (width 0.35) (layer "F.Cu") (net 23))
 (segment (start 147.94 99.45) (end 152.082 103.592) (width 0.35) (layer "F.Cu") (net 23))
 (segment (start 145.16 92.34) (end 145.42 92.34) (width 0.35) (layer "F.Cu") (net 23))
 (segment (start 149.15 94.82) (end 145.4 91.07) (width 0.35) (layer "F.Cu") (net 24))
 (segment (start 151.568 101.228) (end 149.15 98.81) (width 0.35) (layer "F.Cu") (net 24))
 (segment (start 149.15 98.81) (end 149.15 94.82) (width 0.35) (layer "F.Cu") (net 24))
 (segment (start 145.4 91.07) (end 145.16 91.07) (width 0.35) (layer "F.Cu") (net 24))
 (segment (start 152.082 101.228) (end 151.568 101.228) (width 0.35) (layer "F.Cu") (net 24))
 (segment (start 145.16 89.8) (end 145.26 89.8) (width 0.35) (layer "F.Cu") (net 25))
 (segment (start 149.79 94.33) (end 149.79 95.92) (width 0.35) (layer "F.Cu") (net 25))
 (segment (start 149.79 95.92) (end 152.082 98.212) (width 0.35) (layer "F.Cu") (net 25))
 (segment (start 152.082 98.212) (end 152.082 98.688) (width 0.35) (layer "F.Cu") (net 25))
 (segment (start 145.26 89.8) (end 149.79 94.33) (width 0.35) (layer "F.Cu") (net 25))
 (segment (start 150.51 94.53) (end 150.51 93.58) (width 0.35) (layer "F.Cu") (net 26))
 (segment (start 152.082 96.102) (end 150.51 94.53) (width 0.35) (layer "F.Cu") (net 26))
 (segment (start 150.51 93.58) (end 145.46 88.53) (width 0.35) (layer "F.Cu") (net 26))
 (segment (start 152.082 96.148) (end 152.082 96.102) (width 0.35) (layer "F.Cu") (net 26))
 (segment (start 145.46 88.53) (end 145.16 88.53) (width 0.35) (layer "F.Cu") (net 26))
 (segment (start 152.082 93.608) (end 152.082 93.3319) (width 0.35) (layer "F.Cu") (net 27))
 (segment (start 146.0101 87.26) (end 145.16 87.26) (width 0.35) (layer "F.Cu") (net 27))
 (segment (start 152.082 93.3319) (end 146.0101 87.26) (width 0.35) (layer "F.Cu") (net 27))
 (segment (start 151.398 91.068) (end 146.32 85.99) (width 0.35) (layer "F.Cu") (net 28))
 (segment (start 146.32 85.99) (end 145.16 85.99) (width 0.35) (layer "F.Cu") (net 28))
 (segment (start 152.082 91.068) (end 151.398 91.068) (width 0.35) (layer "F.Cu") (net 28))
 (segment (start 147.0739 84.72) (end 150.8819 88.528) (width 0.35) (layer "F.Cu") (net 29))
 (segment (start 145.16 84.72) (end 147.0739 84.72) (width 0.35) (layer "F.Cu") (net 29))
 (segment (start 152.082 88.528) (end 150.8819 88.528) (width 0.35) (layer "F.Cu") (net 29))
 (segment (start 150.8819 85.988) (end 148.3439 83.45) (width 0.35) (layer "F.Cu") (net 30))
 (segment (start 148.3439 83.45) (end 145.16 83.45) (width 0.35) (layer "F.Cu") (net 30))
 (segment (start 152.082 85.988) (end 150.8819 85.988) (width 0.35) (layer "F.Cu") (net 30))
 (segment (start 150.8819 83.448) (end 149.6139 82.18) (width 0.35) (layer "F.Cu") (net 31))
 (segment (start 152.082 83.448) (end 150.8819 83.448) (width 0.35) (layer "F.Cu") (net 31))
 (segment (start 149.6139 82.18) (end 145.16 82.18) (width 0.35) (layer "F.Cu") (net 31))
 (segment (start 146.0121 80.908) (end 146.0101 80.91) (width 0.35) (layer "F.Cu") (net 32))
 (segment (start 152.082 80.908) (end 146.0121 80.908) (width 0.35) (layer "F.Cu") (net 32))
 (segment (start 145.16 80.91) (end 146.0101 80.91) (width 0.35) (layer "F.Cu") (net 32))
 (segment (start 150.8819 78.368) (end 149.6099 79.64) (width 0.35) (layer "F.Cu") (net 33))
 (segment (start 152.082 78.368) (end 150.8819 78.368) (width 0.35) (layer "F.Cu") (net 33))
 (segment (start 149.6099 79.64) (end 145.16 79.64) (width 0.35) (layer "F.Cu") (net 33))
 (segment (start 150.8819 75.828) (end 148.3399 78.37) (width 0.35) (layer "F.Cu") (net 34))
 (segment (start 148.3399 78.37) (end 145.16 78.37) (width 0.35) (layer "F.Cu") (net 34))
 (segment (start 152.082 75.828) (end 150.8819 75.828) (width 0.35) (layer "F.Cu") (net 34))
 (segment (start 145.16 77.1) (end 146.73 77.1) (width 0.35) (layer "F.Cu") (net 35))
 (segment (start 150.542 73.288) (end 152.082 73.288) (width 0.35) (layer "F.Cu") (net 35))
 (segment (start 146.73 77.1) (end 150.542 73.288) (width 0.35) (layer "F.Cu") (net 35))
 (segment (start 146.0101 75.83) (end 145.16 75.83) (width 0.35) (layer "F.Cu") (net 36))
 (segment (start 151.0921 70.748) (end 146.0101 75.83) (width 0.35) (layer "F.Cu") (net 36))
 (segment (start 152.082 70.748) (end 151.0921 70.748) (width 0.35) (layer "F.Cu") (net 36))
 (segment (start 152.082 68.208) (end 151.512 68.208) (width 0.35) (layer "F.Cu") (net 37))
 (segment (start 151.512 68.208) (end 145.16 74.56) (width 0.35) (layer "F.Cu") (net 37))
 (segment (start 146.0775 72.285) (end 146.0775 72.3725) (width 0.35) (layer "F.Cu") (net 38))
 (segment (start 152.082 66.2805) (end 146.0775 72.285) (width 0.35) (layer "F.Cu") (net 38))
 (segment (start 152.082 65.668) (end 152.082 66.2805) (width 0.35) (layer "F.Cu") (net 38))
 (segment (start 146.0775 72.3725) (end 145.16 73.29) (width 0.35) (layer "F.Cu") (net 38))
 (segment (start 152.082 63.248) (end 149.81 65.52) (width 0.35) (layer "F.Cu") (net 39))
 (segment (start 149.81 67.37) (end 145.16 72.02) (width 0.35) (layer "F.Cu") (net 39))
 (segment (start 152.082 63.128) (end 152.082 63.248) (width 0.35) (layer "F.Cu") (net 39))
 (segment (start 149.81 65.52) (end 149.81 67.37) (width 0.35) (layer "F.Cu") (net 39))
 (segment (start 147.27 68.64) (end 147.27 65.38) (width 0.35) (layer "F.Cu") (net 40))
 (segment (start 152.062 60.588) (end 152.082 60.588) (width 0.35) (layer "F.Cu") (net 40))
 (segment (start 147.27 65.38) (end 152.062 60.588) (width 0.35) (layer "F.Cu") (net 40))
 (segment (start 145.16 70.75) (end 147.27 68.64) (width 0.35) (layer "F.Cu") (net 40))
 (segment (start 145.16 69.48) (end 145.43 69.48) (width 0.35) (layer "F.Cu") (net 41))
 (segment (start 146.32 63.82) (end 152.082 58.058) (width 0.35) (layer "F.Cu") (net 41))
 (segment (start 145.43 69.48) (end 146.32 68.59) (width 0.35) (layer "F.Cu") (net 41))
 (segment (start 152.082 58.058) (end 152.082 58.048) (width 0.35) (layer "F.Cu") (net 41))
 (segment (start 146.32 68.59) (end 146.32 63.82) (width 0.35) (layer "F.Cu") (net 41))
 (segment (start 151.922 55.508) (end 145.16 62.27) (width 0.35) (layer "F.Cu") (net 42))
 (segment (start 152.082 55.508) (end 151.922 55.508) (width 0.35) (layer "F.Cu") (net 42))
 (segment (start 145.16 62.27) (end 145.16 68.21) (width 0.35) (layer "F.Cu") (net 42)))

